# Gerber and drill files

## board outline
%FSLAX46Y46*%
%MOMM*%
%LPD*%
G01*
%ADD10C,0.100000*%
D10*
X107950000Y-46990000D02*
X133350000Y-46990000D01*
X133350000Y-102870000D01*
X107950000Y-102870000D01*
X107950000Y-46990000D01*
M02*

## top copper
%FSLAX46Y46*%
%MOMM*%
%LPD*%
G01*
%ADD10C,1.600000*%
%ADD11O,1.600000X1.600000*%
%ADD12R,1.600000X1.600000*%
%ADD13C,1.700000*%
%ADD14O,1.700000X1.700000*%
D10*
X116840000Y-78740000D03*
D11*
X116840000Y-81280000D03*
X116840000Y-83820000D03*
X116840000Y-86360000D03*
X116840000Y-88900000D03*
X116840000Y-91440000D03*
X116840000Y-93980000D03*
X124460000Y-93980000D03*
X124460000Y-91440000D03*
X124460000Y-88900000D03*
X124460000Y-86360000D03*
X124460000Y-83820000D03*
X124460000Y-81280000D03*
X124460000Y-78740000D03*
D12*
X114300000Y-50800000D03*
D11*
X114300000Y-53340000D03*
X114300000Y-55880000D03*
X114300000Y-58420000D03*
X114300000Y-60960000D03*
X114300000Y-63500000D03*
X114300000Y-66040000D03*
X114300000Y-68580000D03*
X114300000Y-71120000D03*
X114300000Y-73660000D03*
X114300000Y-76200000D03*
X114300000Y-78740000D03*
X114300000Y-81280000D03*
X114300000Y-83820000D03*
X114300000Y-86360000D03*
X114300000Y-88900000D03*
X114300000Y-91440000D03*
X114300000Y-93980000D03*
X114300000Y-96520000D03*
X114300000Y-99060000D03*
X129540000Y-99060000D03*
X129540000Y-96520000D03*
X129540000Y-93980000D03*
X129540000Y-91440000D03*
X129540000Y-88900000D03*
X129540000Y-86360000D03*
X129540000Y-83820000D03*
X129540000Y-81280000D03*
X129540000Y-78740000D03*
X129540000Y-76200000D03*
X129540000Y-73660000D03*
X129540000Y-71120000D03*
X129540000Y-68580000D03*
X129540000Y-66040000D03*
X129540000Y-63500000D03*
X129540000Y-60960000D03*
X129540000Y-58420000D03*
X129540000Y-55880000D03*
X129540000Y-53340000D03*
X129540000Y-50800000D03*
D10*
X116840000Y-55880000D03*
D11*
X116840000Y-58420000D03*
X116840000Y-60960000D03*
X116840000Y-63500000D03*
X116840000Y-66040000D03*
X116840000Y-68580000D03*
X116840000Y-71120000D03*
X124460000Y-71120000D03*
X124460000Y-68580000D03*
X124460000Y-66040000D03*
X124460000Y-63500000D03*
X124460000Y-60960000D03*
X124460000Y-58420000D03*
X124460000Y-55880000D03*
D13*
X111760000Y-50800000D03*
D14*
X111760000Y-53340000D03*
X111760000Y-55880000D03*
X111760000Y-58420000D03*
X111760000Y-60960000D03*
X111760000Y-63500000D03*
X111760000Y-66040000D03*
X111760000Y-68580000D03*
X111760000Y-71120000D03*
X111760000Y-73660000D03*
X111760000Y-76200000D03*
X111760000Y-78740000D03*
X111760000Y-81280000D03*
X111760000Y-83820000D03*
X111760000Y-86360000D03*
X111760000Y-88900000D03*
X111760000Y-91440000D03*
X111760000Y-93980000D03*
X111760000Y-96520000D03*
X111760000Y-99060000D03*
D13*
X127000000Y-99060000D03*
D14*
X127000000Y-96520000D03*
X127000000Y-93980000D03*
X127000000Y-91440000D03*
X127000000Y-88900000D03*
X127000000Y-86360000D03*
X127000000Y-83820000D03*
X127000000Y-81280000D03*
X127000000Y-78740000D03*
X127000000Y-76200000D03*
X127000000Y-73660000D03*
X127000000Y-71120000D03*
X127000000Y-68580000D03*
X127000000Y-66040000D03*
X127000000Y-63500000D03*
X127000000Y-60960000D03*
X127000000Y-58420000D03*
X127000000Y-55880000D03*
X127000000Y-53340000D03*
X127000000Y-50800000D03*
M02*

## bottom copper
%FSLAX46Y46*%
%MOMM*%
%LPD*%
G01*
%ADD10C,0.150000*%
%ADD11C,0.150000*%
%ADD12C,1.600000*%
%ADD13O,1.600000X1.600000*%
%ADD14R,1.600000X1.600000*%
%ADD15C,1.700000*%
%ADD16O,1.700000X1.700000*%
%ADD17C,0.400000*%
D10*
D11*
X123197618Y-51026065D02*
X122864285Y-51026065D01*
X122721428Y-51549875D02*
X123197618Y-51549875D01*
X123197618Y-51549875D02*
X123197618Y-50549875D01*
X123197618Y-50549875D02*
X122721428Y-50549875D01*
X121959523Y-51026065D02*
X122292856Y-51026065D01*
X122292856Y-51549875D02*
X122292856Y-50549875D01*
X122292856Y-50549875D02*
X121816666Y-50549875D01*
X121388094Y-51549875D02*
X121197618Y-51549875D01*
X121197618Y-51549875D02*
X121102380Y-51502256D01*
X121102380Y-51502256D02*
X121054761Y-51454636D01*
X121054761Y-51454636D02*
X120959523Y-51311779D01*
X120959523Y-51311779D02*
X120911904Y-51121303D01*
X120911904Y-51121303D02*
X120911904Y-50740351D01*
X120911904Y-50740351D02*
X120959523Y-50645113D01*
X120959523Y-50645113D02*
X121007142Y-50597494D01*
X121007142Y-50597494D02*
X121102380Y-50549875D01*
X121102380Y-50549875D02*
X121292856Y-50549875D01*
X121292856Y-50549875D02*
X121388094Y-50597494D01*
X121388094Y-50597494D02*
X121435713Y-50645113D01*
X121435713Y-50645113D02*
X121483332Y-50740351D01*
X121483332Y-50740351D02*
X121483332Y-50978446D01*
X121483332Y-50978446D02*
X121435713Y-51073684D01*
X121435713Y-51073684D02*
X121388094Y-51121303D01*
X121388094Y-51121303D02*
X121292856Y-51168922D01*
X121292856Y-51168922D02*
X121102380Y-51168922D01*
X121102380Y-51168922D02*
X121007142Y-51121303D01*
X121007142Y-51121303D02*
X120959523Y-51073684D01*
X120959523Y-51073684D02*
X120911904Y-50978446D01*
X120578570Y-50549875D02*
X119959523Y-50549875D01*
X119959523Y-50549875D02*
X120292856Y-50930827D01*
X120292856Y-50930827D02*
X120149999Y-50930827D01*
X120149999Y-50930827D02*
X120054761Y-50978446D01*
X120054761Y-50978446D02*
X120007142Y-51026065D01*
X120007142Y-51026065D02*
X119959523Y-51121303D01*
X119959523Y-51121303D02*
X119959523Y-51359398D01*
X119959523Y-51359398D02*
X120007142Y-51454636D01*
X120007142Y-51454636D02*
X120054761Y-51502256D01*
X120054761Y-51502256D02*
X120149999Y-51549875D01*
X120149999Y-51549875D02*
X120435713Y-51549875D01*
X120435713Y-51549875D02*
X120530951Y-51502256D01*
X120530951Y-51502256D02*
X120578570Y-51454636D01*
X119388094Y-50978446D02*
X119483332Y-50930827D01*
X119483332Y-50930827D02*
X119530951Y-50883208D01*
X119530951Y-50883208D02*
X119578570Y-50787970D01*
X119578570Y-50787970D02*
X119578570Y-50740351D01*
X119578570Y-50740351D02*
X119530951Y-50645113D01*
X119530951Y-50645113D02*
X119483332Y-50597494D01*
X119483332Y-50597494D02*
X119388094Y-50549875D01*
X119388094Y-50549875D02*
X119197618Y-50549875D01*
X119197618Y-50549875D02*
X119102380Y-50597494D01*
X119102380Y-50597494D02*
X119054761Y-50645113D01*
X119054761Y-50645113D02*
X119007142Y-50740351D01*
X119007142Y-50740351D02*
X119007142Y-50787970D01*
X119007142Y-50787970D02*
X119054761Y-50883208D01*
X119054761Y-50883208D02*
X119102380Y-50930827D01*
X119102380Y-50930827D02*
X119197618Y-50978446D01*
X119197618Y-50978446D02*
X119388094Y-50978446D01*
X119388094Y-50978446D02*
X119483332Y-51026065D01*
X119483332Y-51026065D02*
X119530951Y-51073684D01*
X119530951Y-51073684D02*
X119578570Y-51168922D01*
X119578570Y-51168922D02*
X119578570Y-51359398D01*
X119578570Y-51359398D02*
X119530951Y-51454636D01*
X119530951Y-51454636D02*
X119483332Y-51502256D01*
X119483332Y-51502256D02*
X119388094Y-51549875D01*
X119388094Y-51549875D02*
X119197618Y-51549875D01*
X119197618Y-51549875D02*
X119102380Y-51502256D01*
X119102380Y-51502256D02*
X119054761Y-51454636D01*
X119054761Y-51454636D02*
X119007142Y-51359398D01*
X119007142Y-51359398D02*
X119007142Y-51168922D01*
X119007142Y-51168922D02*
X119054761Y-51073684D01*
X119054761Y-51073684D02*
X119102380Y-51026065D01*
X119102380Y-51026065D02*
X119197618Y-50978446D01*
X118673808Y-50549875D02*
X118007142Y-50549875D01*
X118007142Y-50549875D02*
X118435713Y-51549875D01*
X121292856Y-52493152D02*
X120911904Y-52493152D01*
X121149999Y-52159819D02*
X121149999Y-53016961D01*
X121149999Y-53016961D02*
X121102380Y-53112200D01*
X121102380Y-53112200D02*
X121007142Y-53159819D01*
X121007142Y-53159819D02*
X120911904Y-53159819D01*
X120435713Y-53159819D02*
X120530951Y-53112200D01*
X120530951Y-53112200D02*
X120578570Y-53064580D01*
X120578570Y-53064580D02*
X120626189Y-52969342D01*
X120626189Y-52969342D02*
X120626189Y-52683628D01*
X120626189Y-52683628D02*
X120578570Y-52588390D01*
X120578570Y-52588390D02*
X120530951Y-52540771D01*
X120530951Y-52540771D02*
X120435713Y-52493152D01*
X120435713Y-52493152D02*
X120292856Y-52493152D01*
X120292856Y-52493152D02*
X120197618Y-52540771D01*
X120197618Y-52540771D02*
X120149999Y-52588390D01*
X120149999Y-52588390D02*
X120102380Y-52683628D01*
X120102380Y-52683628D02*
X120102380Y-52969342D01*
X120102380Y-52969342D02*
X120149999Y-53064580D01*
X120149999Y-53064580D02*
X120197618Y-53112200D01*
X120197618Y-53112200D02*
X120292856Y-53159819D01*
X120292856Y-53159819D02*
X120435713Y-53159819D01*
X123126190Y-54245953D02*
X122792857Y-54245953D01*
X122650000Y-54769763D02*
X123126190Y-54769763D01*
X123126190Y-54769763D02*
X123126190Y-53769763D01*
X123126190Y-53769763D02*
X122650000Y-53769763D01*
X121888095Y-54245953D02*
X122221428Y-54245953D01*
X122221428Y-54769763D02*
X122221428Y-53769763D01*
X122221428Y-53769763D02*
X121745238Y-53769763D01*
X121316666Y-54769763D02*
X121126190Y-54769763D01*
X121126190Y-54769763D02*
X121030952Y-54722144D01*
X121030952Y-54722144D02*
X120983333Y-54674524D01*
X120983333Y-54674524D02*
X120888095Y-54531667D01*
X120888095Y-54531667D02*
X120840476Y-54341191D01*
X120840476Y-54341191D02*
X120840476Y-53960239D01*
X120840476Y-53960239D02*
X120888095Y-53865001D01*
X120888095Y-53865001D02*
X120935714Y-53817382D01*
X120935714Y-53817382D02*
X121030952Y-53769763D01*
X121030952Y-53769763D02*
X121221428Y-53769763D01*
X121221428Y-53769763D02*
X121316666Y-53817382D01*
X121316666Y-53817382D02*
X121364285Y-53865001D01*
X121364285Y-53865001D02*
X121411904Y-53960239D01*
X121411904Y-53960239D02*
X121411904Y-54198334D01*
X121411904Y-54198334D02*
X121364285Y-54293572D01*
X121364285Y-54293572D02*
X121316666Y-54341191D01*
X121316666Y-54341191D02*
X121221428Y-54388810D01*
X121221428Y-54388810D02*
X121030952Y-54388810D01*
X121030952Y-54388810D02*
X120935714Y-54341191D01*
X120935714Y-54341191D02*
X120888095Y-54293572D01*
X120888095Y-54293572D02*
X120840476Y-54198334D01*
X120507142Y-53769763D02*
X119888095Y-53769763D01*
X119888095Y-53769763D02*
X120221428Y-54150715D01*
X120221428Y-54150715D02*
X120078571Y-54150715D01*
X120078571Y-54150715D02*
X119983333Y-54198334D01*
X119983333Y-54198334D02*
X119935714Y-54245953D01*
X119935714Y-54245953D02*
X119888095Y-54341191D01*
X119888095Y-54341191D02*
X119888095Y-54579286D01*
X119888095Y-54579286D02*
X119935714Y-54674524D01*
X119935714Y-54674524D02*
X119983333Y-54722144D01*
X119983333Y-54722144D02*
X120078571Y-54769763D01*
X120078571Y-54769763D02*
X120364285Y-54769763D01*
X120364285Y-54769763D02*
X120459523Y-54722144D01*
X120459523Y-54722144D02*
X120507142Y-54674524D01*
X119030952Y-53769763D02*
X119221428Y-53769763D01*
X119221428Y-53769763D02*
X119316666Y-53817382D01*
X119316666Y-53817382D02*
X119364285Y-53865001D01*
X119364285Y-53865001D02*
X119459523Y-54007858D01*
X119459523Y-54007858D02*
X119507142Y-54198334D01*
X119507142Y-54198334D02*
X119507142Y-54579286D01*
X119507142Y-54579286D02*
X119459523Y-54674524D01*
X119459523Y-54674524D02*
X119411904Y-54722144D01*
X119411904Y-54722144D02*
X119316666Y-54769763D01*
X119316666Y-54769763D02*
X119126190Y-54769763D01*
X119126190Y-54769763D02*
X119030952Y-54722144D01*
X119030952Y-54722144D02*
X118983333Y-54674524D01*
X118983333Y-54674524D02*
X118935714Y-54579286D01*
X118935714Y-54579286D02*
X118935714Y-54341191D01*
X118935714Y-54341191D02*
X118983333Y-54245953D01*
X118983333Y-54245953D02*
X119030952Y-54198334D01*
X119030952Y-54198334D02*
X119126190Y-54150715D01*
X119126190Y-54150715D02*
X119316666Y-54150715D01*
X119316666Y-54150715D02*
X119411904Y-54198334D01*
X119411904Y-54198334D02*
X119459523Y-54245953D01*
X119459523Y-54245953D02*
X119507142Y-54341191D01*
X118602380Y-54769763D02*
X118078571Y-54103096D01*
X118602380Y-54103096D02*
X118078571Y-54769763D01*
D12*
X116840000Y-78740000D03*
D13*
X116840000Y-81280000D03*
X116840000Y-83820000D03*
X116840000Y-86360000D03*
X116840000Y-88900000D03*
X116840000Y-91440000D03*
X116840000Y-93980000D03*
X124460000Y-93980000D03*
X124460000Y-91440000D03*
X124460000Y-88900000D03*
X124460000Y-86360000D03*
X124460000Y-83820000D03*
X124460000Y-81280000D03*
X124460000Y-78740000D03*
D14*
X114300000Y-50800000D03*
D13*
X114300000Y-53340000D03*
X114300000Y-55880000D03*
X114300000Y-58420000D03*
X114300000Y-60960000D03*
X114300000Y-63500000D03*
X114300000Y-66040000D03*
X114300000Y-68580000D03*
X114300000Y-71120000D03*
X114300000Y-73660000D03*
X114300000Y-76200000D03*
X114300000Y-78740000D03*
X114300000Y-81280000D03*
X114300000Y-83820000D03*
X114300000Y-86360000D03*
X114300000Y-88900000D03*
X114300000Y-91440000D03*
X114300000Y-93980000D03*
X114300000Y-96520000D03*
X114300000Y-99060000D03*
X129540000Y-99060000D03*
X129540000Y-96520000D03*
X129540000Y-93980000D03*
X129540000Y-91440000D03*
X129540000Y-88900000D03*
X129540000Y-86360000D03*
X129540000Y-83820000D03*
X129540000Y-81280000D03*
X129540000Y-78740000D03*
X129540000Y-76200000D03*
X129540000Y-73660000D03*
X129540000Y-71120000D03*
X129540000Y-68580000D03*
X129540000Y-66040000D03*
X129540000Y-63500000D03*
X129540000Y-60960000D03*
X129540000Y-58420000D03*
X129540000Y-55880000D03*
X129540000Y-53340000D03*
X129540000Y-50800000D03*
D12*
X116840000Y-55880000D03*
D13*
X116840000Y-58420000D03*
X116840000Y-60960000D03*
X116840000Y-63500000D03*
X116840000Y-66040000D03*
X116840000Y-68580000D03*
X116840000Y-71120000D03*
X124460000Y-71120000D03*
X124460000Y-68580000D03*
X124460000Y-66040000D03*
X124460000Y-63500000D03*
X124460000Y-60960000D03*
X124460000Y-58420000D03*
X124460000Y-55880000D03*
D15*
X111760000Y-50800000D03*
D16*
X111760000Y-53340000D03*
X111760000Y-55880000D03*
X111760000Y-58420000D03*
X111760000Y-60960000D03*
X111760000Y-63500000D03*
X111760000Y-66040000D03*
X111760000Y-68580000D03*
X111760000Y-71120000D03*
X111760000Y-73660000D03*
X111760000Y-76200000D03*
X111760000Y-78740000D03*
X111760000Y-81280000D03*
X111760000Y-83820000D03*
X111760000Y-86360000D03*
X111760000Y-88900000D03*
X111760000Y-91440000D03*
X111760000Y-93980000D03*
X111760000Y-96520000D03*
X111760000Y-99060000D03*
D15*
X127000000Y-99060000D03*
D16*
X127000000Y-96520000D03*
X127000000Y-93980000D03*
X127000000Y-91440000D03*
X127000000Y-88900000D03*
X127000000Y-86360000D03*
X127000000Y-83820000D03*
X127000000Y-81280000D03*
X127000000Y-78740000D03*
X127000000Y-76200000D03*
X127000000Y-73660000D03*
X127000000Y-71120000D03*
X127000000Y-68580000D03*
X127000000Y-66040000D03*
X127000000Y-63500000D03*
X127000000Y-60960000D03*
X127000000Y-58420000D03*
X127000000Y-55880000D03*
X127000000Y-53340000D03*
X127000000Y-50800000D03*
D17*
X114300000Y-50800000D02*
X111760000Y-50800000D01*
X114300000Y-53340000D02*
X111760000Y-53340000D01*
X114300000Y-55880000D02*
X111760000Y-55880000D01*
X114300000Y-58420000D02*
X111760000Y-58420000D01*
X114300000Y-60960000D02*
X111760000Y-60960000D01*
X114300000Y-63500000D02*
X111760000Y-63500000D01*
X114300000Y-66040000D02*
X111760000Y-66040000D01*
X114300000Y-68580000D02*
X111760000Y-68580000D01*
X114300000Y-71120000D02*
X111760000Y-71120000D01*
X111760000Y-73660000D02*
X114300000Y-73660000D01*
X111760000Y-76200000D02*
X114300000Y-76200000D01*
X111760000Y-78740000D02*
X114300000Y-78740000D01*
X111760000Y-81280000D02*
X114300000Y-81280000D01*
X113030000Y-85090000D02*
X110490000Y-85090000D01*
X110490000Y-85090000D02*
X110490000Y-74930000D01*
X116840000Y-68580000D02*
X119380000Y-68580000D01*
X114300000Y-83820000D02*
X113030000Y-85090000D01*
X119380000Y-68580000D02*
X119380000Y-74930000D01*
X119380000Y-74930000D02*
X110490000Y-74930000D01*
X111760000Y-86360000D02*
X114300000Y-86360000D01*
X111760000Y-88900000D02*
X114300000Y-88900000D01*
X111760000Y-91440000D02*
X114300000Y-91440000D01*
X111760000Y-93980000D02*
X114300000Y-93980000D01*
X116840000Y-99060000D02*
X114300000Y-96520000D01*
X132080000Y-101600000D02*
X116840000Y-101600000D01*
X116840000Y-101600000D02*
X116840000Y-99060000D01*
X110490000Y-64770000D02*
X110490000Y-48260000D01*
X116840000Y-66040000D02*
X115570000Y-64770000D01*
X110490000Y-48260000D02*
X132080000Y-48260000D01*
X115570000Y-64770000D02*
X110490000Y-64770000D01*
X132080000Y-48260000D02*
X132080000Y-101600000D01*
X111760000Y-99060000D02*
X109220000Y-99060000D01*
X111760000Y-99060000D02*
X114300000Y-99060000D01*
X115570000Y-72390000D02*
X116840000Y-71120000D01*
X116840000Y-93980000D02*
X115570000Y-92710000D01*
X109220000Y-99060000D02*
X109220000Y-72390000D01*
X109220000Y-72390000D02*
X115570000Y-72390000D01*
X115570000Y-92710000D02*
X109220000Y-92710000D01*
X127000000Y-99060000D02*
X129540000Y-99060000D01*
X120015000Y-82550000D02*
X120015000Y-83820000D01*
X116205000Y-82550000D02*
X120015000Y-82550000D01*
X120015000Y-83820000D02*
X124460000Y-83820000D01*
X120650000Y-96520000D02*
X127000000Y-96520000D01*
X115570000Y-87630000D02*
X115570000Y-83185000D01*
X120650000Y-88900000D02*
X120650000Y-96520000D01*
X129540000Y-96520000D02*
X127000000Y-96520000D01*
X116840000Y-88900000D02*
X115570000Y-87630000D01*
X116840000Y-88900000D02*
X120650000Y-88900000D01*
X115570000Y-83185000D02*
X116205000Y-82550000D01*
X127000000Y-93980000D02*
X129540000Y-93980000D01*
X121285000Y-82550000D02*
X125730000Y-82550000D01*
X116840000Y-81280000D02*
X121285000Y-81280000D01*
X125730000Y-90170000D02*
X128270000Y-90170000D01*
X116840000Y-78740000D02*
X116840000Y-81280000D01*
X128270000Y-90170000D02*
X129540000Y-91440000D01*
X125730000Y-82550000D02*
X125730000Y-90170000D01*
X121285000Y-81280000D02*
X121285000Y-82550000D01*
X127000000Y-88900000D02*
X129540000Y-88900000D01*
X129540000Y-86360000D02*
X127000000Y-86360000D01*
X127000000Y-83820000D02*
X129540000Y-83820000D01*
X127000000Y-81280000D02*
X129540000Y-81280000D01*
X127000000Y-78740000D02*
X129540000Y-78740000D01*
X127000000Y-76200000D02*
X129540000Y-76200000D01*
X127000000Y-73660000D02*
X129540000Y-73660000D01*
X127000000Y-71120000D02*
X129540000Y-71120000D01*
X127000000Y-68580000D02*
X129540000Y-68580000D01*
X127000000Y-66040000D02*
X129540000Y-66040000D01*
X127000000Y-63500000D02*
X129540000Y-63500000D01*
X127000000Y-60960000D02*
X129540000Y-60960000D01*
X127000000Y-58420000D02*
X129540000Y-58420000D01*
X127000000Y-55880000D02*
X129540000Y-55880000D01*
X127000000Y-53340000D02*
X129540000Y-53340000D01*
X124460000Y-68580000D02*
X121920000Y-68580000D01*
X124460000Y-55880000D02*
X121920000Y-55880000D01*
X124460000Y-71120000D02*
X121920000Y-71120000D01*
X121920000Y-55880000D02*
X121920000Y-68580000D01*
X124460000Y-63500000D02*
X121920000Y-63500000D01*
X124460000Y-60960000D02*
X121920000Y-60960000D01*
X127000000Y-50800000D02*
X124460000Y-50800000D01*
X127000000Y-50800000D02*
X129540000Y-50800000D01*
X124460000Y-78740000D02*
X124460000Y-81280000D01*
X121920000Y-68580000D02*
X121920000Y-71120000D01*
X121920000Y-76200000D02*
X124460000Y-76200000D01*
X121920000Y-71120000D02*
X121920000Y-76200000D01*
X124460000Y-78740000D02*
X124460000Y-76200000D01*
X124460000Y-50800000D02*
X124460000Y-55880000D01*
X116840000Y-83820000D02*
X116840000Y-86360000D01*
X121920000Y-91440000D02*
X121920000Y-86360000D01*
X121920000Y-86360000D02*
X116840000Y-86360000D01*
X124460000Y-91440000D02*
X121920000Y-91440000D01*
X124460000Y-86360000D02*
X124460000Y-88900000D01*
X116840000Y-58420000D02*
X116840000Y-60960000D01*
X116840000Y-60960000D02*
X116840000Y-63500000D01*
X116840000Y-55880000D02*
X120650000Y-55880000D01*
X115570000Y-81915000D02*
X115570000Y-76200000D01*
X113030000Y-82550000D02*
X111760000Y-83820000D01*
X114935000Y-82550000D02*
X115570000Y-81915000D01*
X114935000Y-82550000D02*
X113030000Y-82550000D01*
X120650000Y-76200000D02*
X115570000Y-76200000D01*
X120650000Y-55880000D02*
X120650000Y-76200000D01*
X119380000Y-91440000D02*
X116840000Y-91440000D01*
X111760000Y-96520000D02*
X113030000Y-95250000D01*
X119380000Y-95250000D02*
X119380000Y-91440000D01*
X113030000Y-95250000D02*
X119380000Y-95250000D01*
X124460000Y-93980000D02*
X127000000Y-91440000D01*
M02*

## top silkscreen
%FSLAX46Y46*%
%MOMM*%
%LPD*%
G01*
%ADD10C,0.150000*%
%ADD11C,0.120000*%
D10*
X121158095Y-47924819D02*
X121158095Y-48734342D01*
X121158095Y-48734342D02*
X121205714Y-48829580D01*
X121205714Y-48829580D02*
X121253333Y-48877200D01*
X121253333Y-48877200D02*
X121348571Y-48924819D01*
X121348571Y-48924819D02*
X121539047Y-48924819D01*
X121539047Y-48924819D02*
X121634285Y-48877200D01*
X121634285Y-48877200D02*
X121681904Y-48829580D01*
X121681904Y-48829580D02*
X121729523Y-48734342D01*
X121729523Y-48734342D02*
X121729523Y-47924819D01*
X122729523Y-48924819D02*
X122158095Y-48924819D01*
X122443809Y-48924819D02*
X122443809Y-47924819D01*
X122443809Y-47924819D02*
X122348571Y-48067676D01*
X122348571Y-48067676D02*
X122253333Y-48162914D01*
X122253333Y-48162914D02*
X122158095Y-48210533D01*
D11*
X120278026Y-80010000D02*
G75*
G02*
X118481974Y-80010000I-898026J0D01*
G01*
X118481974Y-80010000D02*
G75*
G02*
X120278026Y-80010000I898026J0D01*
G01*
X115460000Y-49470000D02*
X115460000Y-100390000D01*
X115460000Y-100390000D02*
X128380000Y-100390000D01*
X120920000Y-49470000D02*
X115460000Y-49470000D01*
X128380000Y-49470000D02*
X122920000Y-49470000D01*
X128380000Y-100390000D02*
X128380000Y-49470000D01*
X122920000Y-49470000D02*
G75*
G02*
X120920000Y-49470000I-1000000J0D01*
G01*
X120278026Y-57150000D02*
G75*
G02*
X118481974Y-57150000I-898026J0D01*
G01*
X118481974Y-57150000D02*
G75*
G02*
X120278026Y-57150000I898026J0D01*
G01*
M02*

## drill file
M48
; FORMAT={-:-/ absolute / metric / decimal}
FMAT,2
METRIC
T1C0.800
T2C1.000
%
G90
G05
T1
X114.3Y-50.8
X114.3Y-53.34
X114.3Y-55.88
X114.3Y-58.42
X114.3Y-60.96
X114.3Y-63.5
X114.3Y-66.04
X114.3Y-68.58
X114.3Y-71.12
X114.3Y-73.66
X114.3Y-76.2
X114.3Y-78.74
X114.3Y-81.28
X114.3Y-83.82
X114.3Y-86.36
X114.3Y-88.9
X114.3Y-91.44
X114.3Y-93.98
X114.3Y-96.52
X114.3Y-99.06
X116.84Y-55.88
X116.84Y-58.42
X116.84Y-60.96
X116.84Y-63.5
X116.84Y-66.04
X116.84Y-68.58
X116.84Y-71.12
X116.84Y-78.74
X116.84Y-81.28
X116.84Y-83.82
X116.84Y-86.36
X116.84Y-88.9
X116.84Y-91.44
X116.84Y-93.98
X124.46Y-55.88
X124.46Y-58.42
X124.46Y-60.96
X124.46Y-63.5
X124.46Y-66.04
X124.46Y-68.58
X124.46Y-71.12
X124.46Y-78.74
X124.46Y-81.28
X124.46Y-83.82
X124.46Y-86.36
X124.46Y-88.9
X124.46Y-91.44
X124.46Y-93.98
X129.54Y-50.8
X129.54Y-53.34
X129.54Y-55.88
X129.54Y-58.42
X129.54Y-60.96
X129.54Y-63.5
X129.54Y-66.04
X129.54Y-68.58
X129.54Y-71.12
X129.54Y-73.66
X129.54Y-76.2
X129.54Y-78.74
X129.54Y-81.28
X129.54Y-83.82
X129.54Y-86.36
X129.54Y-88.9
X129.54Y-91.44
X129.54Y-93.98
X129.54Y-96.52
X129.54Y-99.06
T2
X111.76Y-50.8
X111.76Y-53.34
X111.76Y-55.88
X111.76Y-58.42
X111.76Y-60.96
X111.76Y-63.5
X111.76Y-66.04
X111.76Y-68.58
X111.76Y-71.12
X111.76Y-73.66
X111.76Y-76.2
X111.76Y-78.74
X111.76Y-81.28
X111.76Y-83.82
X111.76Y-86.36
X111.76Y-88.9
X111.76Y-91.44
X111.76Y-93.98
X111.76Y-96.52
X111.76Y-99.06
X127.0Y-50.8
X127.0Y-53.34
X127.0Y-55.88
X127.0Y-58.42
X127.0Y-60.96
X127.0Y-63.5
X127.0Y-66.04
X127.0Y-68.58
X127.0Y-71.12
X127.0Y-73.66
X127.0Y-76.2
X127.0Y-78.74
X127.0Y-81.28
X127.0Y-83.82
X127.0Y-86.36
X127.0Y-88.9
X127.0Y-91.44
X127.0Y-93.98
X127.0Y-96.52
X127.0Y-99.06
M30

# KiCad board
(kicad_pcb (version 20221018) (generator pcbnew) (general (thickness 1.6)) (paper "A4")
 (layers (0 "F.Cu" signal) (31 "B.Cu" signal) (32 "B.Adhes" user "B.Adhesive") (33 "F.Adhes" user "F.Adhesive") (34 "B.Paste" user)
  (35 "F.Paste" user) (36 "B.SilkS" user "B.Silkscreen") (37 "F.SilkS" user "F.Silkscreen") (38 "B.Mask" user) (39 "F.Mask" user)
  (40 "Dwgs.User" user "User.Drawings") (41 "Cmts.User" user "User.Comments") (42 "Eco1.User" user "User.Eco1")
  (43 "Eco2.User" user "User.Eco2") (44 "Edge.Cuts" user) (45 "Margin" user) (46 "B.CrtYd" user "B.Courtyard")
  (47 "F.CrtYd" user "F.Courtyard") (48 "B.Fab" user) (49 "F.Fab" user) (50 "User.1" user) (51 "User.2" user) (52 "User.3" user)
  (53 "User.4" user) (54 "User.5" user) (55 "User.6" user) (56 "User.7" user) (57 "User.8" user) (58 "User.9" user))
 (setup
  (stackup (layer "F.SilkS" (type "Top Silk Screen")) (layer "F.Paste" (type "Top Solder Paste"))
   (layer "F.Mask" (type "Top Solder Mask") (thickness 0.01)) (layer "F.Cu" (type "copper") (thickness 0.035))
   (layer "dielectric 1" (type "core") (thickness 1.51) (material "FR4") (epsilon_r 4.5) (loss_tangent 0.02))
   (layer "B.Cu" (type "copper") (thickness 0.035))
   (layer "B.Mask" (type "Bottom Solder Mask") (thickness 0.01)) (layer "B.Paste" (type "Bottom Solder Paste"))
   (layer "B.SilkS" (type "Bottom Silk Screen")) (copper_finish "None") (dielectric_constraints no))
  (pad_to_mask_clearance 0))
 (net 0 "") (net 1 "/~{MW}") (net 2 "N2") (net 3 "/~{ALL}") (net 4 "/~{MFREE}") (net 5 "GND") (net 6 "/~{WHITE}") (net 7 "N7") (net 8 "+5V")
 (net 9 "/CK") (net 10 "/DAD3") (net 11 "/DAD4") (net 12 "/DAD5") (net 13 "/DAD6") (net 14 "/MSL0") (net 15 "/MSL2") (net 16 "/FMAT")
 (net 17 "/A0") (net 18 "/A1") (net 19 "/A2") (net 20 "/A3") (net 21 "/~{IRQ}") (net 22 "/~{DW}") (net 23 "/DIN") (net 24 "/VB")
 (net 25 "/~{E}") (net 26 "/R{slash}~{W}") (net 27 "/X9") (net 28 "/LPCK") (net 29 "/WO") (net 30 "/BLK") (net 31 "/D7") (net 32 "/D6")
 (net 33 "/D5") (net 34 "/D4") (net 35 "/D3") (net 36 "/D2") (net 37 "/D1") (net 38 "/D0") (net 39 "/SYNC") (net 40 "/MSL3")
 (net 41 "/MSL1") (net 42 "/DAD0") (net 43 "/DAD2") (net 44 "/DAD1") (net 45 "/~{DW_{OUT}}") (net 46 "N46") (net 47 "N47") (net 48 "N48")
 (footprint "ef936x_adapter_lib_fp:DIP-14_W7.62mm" (layer "F.Cu") (at 116.84 78.74)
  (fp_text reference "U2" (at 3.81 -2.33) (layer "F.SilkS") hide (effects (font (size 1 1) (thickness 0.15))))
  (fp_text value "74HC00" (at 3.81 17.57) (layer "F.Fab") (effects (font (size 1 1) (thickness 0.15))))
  (fp_circle (center 2.54 1.27) (end 3.438026 1.27) (stroke (width 0.12) (type solid)) (fill none) (layer "F.SilkS"))
  (pad "1" thru_hole circle (at 0 0) (size 1.6 1.6) (drill 0.8) (layers "*.Cu" "*.Mask") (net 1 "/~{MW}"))
  (pad "2" thru_hole oval (at 0 2.54) (size 1.6 1.6) (drill 0.8) (layers "*.Cu" "*.Mask") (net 1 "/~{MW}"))
  (pad "3" thru_hole oval (at 0 5.08) (size 1.6 1.6) (drill 0.8) (layers "*.Cu" "*.Mask") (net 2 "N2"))
  (pad "4" thru_hole oval (at 0 7.62) (size 1.6 1.6) (drill 0.8) (layers "*.Cu" "*.Mask") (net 2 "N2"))
  (pad "5" thru_hole oval (at 0 10.16) (size 1.6 1.6) (drill 0.8) (layers "*.Cu" "*.Mask") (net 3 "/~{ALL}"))
  (pad "6" thru_hole oval (at 0 12.7) (size 1.6 1.6) (drill 0.8) (layers "*.Cu" "*.Mask") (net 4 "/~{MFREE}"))
  (pad "7" thru_hole oval (at 0 15.24) (size 1.6 1.6) (drill 0.8) (layers "*.Cu" "*.Mask") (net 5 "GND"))
  (pad "8" thru_hole oval (at 7.62 15.24) (size 1.6 1.6) (drill 0.8) (layers "*.Cu" "*.Mask") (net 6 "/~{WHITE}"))
  (pad "9" thru_hole oval (at 7.62 12.7) (size 1.6 1.6) (drill 0.8) (layers "*.Cu" "*.Mask") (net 2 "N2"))
  (pad "10" thru_hole oval (at 7.62 10.16) (size 1.6 1.6) (drill 0.8) (layers "*.Cu" "*.Mask") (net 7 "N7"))
  (pad "11" thru_hole oval (at 7.62 7.62) (size 1.6 1.6) (drill 0.8) (layers "*.Cu" "*.Mask") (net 7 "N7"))
  (pad "12" thru_hole oval (at 7.62 5.08) (size 1.6 1.6) (drill 0.8) (layers "*.Cu" "*.Mask") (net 3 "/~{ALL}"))
  (pad "13" thru_hole oval (at 7.62 2.54) (size 1.6 1.6) (drill 0.8) (layers "*.Cu" "*.Mask") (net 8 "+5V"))
  (pad "14" thru_hole oval (at 7.62 0) (size 1.6 1.6) (drill 0.8) (layers "*.Cu" "*.Mask") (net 8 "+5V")))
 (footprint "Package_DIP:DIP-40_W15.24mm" (layer "F.Cu") (at 114.3 50.8)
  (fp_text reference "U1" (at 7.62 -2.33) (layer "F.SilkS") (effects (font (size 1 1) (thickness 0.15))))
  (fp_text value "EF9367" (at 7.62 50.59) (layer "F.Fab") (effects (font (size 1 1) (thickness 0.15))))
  (fp_line (start 1.16 -1.33) (end 1.16 49.59) (stroke (width 0.12) (type solid)) (layer "F.SilkS"))
  (fp_line (start 1.16 49.59) (end 14.08 49.59) (stroke (width 0.12) (type solid)) (layer "F.SilkS"))
  (fp_line (start 6.62 -1.33) (end 1.16 -1.33) (stroke (width 0.12) (type solid)) (layer "F.SilkS"))
  (fp_line (start 14.08 -1.33) (end 8.62 -1.33) (stroke (width 0.12) (type solid)) (layer "F.SilkS"))
  (fp_line (start 14.08 49.59) (end 14.08 -1.33) (stroke (width 0.12) (type solid)) (layer "F.SilkS"))
  (fp_arc (start 8.62 -1.33) (mid 7.62 -0.33) (end 6.62 -1.33) (stroke (width 0.12) (type solid)) (layer "F.SilkS"))
  (pad "1" thru_hole rect (at 0 0) (size 1.6 1.6) (drill 0.8) (layers "*.Cu" "*.Mask") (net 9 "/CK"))
  (pad "2" thru_hole oval (at 0 2.54) (size 1.6 1.6) (drill 0.8) (layers "*.Cu" "*.Mask") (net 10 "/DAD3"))
  (pad "3" thru_hole oval (at 0 5.08) (size 1.6 1.6) (drill 0.8) (layers "*.Cu" "*.Mask") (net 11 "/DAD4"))
  (pad "4" thru_hole oval (at 0 7.62) (size 1.6 1.6) (drill 0.8) (layers "*.Cu" "*.Mask") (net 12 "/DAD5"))
  (pad "5" thru_hole oval (at 0 10.16) (size 1.6 1.6) (drill 0.8) (layers "*.Cu" "*.Mask") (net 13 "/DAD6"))
  (pad "6" thru_hole oval (at 0 12.7) (size 1.6 1.6) (drill 0.8) (layers "*.Cu" "*.Mask") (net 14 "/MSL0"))
  (pad "7" thru_hole oval (at 0 15.24) (size 1.6 1.6) (drill 0.8) (layers "*.Cu" "*.Mask") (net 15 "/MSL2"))
  (pad "8" thru_hole oval (at 0 17.78) (size 1.6 1.6) (drill 0.8) (layers "*.Cu" "*.Mask") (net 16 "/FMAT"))
  (pad "9" thru_hole oval (at 0 20.32) (size 1.6 1.6) (drill 0.8) (layers "*.Cu" "*.Mask") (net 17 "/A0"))
  (pad "10" thru_hole oval (at 0 22.86) (size 1.6 1.6) (drill 0.8) (layers "*.Cu" "*.Mask") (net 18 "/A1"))
  (pad "11" thru_hole oval (at 0 25.4) (size 1.6 1.6) (drill 0.8) (layers "*.Cu" "*.Mask") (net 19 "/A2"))
  (pad "12" thru_hole oval (at 0 27.94) (size 1.6 1.6) (drill 0.8) (layers "*.Cu" "*.Mask") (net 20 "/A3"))
  (pad "13" thru_hole oval (at 0 30.48) (size 1.6 1.6) (drill 0.8) (layers "*.Cu" "*.Mask") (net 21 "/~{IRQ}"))
  (pad "14" thru_hole oval (at 0 33.02) (size 1.6 1.6) (drill 0.8) (layers "*.Cu" "*.Mask") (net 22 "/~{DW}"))
  (pad "15" thru_hole oval (at 0 35.56) (size 1.6 1.6) (drill 0.8) (layers "*.Cu" "*.Mask") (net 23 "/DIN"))
  (pad "16" thru_hole oval (at 0 38.1) (size 1.6 1.6) (drill 0.8) (layers "*.Cu" "*.Mask") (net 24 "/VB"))
  (pad "17" thru_hole oval (at 0 40.64) (size 1.6 1.6) (drill 0.8) (layers "*.Cu" "*.Mask") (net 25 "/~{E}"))
  (pad "18" thru_hole oval (at 0 43.18) (size 1.6 1.6) (drill 0.8) (layers "*.Cu" "*.Mask") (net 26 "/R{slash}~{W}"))
  (pad "19" thru_hole oval (at 0 45.72) (size 1.6 1.6) (drill 0.8) (layers "*.Cu" "*.Mask") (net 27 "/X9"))
  (pad "20" thru_hole oval (at 0 48.26) (size 1.6 1.6) (drill 0.8) (layers "*.Cu" "*.Mask") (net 5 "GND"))
  (pad "21" thru_hole oval (at 15.24 48.26) (size 1.6 1.6) (drill 0.8) (layers "*.Cu" "*.Mask") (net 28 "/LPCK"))
  (pad "22" thru_hole oval (at 15.24 45.72) (size 1.6 1.6) (drill 0.8) (layers "*.Cu" "*.Mask") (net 3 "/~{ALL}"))
  (pad "23" thru_hole oval (at 15.24 43.18) (size 1.6 1.6) (drill 0.8) (layers "*.Cu" "*.Mask") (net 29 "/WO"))
  (pad "24" thru_hole oval (at 15.24 40.64) (size 1.6 1.6) (drill 0.8) (layers "*.Cu" "*.Mask") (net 1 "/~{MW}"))
  (pad "25" thru_hole oval (at 15.24 38.1) (size 1.6 1.6) (drill 0.8) (layers "*.Cu" "*.Mask") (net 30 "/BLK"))
  (pad "26" thru_hole oval (at 15.24 35.56) (size 1.6 1.6) (drill 0.8) (layers "*.Cu" "*.Mask") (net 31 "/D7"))
  (pad "27" thru_hole oval (at 15.24 33.02) (size 1.6 1.6) (drill 0.8) (layers "*.Cu" "*.Mask") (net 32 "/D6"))
  (pad "28" thru_hole oval (at 15.24 30.48) (size 1.6 1.6) (drill 0.8) (layers "*.Cu" "*.Mask") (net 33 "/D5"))
  (pad "29" thru_hole oval (at 15.24 27.94) (size 1.6 1.6) (drill 0.8) (layers "*.Cu" "*.Mask") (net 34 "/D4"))
  (pad "30" thru_hole oval (at 15.24 25.4) (size 1.6 1.6) (drill 0.8) (layers "*.Cu" "*.Mask") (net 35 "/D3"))
  (pad "31" thru_hole oval (at 15.24 22.86) (size 1.6 1.6) (drill 0.8) (layers "*.Cu" "*.Mask") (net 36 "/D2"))
  (pad "32" thru_hole oval (at 15.24 20.32) (size 1.6 1.6) (drill 0.8) (layers "*.Cu" "*.Mask") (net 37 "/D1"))
  (pad "33" thru_hole oval (at 15.24 17.78) (size 1.6 1.6) (drill 0.8) (layers "*.Cu" "*.Mask") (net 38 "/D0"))
  (pad "34" thru_hole oval (at 15.24 15.24) (size 1.6 1.6) (drill 0.8) (layers "*.Cu" "*.Mask") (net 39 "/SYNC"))
  (pad "35" thru_hole oval (at 15.24 12.7) (size 1.6 1.6) (drill 0.8) (layers "*.Cu" "*.Mask") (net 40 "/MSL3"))
  (pad "36" thru_hole oval (at 15.24 10.16) (size 1.6 1.6) (drill 0.8) (layers "*.Cu" "*.Mask") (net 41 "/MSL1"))
  (pad "37" thru_hole oval (at 15.24 7.62) (size 1.6 1.6) (drill 0.8) (layers "*.Cu" "*.Mask") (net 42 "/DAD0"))
  (pad "38" thru_hole oval (at 15.24 5.08) (size 1.6 1.6) (drill 0.8) (layers "*.Cu" "*.Mask") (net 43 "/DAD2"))
  (pad "39" thru_hole oval (at 15.24 2.54) (size 1.6 1.6) (drill 0.8) (layers "*.Cu" "*.Mask") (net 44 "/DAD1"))
  (pad "40" thru_hole oval (at 15.24 0) (size 1.6 1.6) (drill 0.8) (layers "*.Cu" "*.Mask") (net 8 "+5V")))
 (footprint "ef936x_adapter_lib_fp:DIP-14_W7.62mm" (layer "F.Cu") (at 116.84 55.88)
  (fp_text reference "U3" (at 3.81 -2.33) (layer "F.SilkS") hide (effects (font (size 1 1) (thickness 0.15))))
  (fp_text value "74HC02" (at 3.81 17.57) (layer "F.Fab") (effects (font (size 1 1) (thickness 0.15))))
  (fp_circle (center 2.54 1.27) (end 3.438026 1.27) (stroke (width 0.12) (type solid)) (fill none) (layer "F.SilkS"))
  (pad "1" thru_hole circle (at 0 0) (size 1.6 1.6) (drill 0.8) (layers "*.Cu" "*.Mask") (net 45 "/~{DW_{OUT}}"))
  (pad "2" thru_hole oval (at 0 2.54) (size 1.6 1.6) (drill 0.8) (layers "*.Cu" "*.Mask") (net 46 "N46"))
  (pad "3" thru_hole oval (at 0 5.08) (size 1.6 1.6) (drill 0.8) (layers "*.Cu" "*.Mask") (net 46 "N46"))
  (pad "4" thru_hole oval (at 0 7.62) (size 1.6 1.6) (drill 0.8) (layers "*.Cu" "*.Mask") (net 46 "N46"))
  (pad "5" thru_hole oval (at 0 10.16) (size 1.6 1.6) (drill 0.8) (layers "*.Cu" "*.Mask") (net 27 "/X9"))
  (pad "6" thru_hole oval (at 0 12.7) (size 1.6 1.6) (drill 0.8) (layers "*.Cu" "*.Mask") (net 22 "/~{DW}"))
  (pad "7" thru_hole oval (at 0 15.24) (size 1.6 1.6) (drill 0.8) (layers "*.Cu" "*.Mask") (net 5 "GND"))
  (pad "8" thru_hole oval (at 7.62 15.24) (size 1.6 1.6) (drill 0.8) (layers "*.Cu" "*.Mask") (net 8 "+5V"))
  (pad "9" thru_hole oval (at 7.62 12.7) (size 1.6 1.6) (drill 0.8) (layers "*.Cu" "*.Mask") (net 8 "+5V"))
  (pad "10" thru_hole oval (at 7.62 10.16) (size 1.6 1.6) (drill 0.8) (layers "*.Cu" "*.Mask") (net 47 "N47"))
  (pad "11" thru_hole oval (at 7.62 7.62) (size 1.6 1.6) (drill 0.8) (layers "*.Cu" "*.Mask") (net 8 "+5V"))
  (pad "12" thru_hole oval (at 7.62 5.08) (size 1.6 1.6) (drill 0.8) (layers "*.Cu" "*.Mask") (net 8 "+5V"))
  (pad "13" thru_hole oval (at 7.62 2.54) (size 1.6 1.6) (drill 0.8) (layers "*.Cu" "*.Mask") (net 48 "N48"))
  (pad "14" thru_hole oval (at 7.62 0) (size 1.6 1.6) (drill 0.8) (layers "*.Cu" "*.Mask") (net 8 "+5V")))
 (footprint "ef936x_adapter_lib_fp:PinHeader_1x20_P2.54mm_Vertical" (layer "B.Cu") (at 111.76 50.8 180)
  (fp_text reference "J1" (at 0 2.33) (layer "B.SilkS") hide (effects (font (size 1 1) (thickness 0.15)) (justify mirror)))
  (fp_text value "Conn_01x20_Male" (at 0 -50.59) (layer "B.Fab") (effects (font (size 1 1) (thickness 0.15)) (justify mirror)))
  (pad "1" thru_hole circle (at 0 0 180) (size 1.7 1.7) (drill 1) (layers "*.Cu" "*.Mask") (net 9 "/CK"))
  (pad "2" thru_hole oval (at 0 -2.54 180) (size 1.7 1.7) (drill 1) (layers "*.Cu" "*.Mask") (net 10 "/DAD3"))
  (pad "3" thru_hole oval (at 0 -5.08 180) (size 1.7 1.7) (drill 1) (layers "*.Cu" "*.Mask") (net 11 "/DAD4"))
  (pad "4" thru_hole oval (at 0 -7.62 180) (size 1.7 1.7) (drill 1) (layers "*.Cu" "*.Mask") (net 12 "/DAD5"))
  (pad "5" thru_hole oval (at 0 -10.16 180) (size 1.7 1.7) (drill 1) (layers "*.Cu" "*.Mask") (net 13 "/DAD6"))
  (pad "6" thru_hole oval (at 0 -12.7 180) (size 1.7 1.7) (drill 1) (layers "*.Cu" "*.Mask") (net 14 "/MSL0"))
  (pad "7" thru_hole oval (at 0 -15.24 180) (size 1.7 1.7) (drill 1) (layers "*.Cu" "*.Mask") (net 15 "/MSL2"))
  (pad "8" thru_hole oval (at 0 -17.78 180) (size 1.7 1.7) (drill 1) (layers "*.Cu" "*.Mask") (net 16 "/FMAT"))
  (pad "9" thru_hole oval (at 0 -20.32 180) (size 1.7 1.7) (drill 1) (layers "*.Cu" "*.Mask") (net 17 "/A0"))
  (pad "10" thru_hole oval (at 0 -22.86 180) (size 1.7 1.7) (drill 1) (layers "*.Cu" "*.Mask") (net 18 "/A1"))
  (pad "11" thru_hole oval (at 0 -25.4 180) (size 1.7 1.7) (drill 1) (layers "*.Cu" "*.Mask") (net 19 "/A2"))
  (pad "12" thru_hole oval (at 0 -27.94 180) (size 1.7 1.7) (drill 1) (layers "*.Cu" "*.Mask") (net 20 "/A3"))
  (pad "13" thru_hole oval (at 0 -30.48 180) (size 1.7 1.7) (drill 1) (layers "*.Cu" "*.Mask") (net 21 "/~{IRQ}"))
  (pad "14" thru_hole oval (at 0 -33.02 180) (size 1.7 1.7) (drill 1) (layers "*.Cu" "*.Mask") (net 45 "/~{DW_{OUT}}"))
  (pad "15" thru_hole oval (at 0 -35.56 180) (size 1.7 1.7) (drill 1) (layers "*.Cu" "*.Mask") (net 23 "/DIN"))
  (pad "16" thru_hole oval (at 0 -38.1 180) (size 1.7 1.7) (drill 1) (layers "*.Cu" "*.Mask") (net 24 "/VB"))
  (pad "17" thru_hole oval (at 0 -40.64 180) (size 1.7 1.7) (drill 1) (layers "*.Cu" "*.Mask") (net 25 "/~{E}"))
  (pad "18" thru_hole oval (at 0 -43.18 180) (size 1.7 1.7) (drill 1) (layers "*.Cu" "*.Mask") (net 26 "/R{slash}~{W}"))
  (pad "19" thru_hole oval (at 0 -45.72 180) (size 1.7 1.7) (drill 1) (layers "*.Cu" "*.Mask") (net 4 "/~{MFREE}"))
  (pad "20" thru_hole oval (at 0 -48.26 180) (size 1.7 1.7) (drill 1) (layers "*.Cu" "*.Mask") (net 5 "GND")))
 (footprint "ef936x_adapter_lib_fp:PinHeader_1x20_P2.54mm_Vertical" (layer "B.Cu") (at 127 99.06)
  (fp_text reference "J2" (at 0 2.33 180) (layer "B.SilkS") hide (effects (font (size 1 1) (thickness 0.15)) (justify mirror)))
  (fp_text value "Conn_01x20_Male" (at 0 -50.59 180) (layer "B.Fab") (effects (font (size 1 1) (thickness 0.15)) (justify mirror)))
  (pad "1" thru_hole circle (at 0 0) (size 1.7 1.7) (drill 1) (layers "*.Cu" "*.Mask") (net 28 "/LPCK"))
  (pad "2" thru_hole oval (at 0 -2.54) (size 1.7 1.7) (drill 1) (layers "*.Cu" "*.Mask") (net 3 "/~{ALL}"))
  (pad "3" thru_hole oval (at 0 -5.08) (size 1.7 1.7) (drill 1) (layers "*.Cu" "*.Mask") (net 29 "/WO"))
  (pad "4" thru_hole oval (at 0 -7.62) (size 1.7 1.7) (drill 1) (layers "*.Cu" "*.Mask") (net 6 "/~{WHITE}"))
  (pad "5" thru_hole oval (at 0 -10.16) (size 1.7 1.7) (drill 1) (layers "*.Cu" "*.Mask") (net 30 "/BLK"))
  (pad "6" thru_hole oval (at 0 -12.7) (size 1.7 1.7) (drill 1) (layers "*.Cu" "*.Mask") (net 31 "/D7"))
  (pad "7" thru_hole oval (at 0 -15.24) (size 1.7 1.7) (drill 1) (layers "*.Cu" "*.Mask") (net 32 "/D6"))
  (pad "8" thru_hole oval (at 0 -17.78) (size 1.7 1.7) (drill 1) (layers "*.Cu" "*.Mask") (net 33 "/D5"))
  (pad "9" thru_hole oval (at 0 -20.32) (size 1.7 1.7) (drill 1) (layers "*.Cu" "*.Mask") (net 34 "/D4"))
  (pad "10" thru_hole oval (at 0 -22.86) (size 1.7 1.7) (drill 1) (layers "*.Cu" "*.Mask") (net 35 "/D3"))
  (pad "11" thru_hole oval (at 0 -25.4) (size 1.7 1.7) (drill 1) (layers "*.Cu" "*.Mask") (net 36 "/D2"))
  (pad "12" thru_hole oval (at 0 -27.94) (size 1.7 1.7) (drill 1) (layers "*.Cu" "*.Mask") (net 37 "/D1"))
  (pad "13" thru_hole oval (at 0 -30.48) (size 1.7 1.7) (drill 1) (layers "*.Cu" "*.Mask") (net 38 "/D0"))
  (pad "14" thru_hole oval (at 0 -33.02) (size 1.7 1.7) (drill 1) (layers "*.Cu" "*.Mask") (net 39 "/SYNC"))
  (pad "15" thru_hole oval (at 0 -35.56) (size 1.7 1.7) (drill 1) (layers "*.Cu" "*.Mask") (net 40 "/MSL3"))
  (pad "16" thru_hole oval (at 0 -38.1) (size 1.7 1.7) (drill 1) (layers "*.Cu" "*.Mask") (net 41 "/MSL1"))
  (pad "17" thru_hole oval (at 0 -40.64) (size 1.7 1.7) (drill 1) (layers "*.Cu" "*.Mask") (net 42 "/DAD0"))
  (pad "18" thru_hole oval (at 0 -43.18) (size 1.7 1.7) (drill 1) (layers "*.Cu" "*.Mask") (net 43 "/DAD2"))
  (pad "19" thru_hole oval (at 0 -45.72) (size 1.7 1.7) (drill 1) (layers "*.Cu" "*.Mask") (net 44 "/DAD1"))
  (pad "20" thru_hole oval (at 0 -48.26) (size 1.7 1.7) (drill 1) (layers "*.Cu" "*.Mask") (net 8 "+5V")))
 (gr_rect (start 107.95 46.99) (end 133.35 102.87) (stroke (width 0.1) (type solid)) (fill none) (layer "Edge.Cuts"))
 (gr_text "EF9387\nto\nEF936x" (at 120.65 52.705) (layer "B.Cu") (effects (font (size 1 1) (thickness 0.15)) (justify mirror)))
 (segment (start 114.3 50.8) (end 111.76 50.8) (width 0.4) (layer "B.Cu") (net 9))
 (segment (start 114.3 53.34) (end 111.76 53.34) (width 0.4) (layer "B.Cu") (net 10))
 (segment (start 114.3 55.88) (end 111.76 55.88) (width 0.4) (layer "B.Cu") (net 11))
 (segment (start 114.3 58.42) (end 111.76 58.42) (width 0.4) (layer "B.Cu") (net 12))
 (segment (start 114.3 60.96) (end 111.76 60.96) (width 0.4) (layer "B.Cu") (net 13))
 (segment (start 114.3 63.5) (end 111.76 63.5) (width 0.4) (layer "B.Cu") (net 14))
 (segment (start 114.3 66.04) (end 111.76 66.04) (width 0.4) (layer "B.Cu") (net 15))
 (segment (start 114.3 68.58) (end 111.76 68.58) (width 0.4) (layer "B.Cu") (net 16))
 (segment (start 114.3 71.12) (end 111.76 71.12) (width 0.4) (layer "B.Cu") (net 17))
 (segment (start 111.76 73.66) (end 114.3 73.66) (width 0.4) (layer "B.Cu") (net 18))
 (segment (start 111.76 76.2) (end 114.3 76.2) (width 0.4) (layer "B.Cu") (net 19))
 (segment (start 111.76 78.74) (end 114.3 78.74) (width 0.4) (layer "B.Cu") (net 20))
 (segment (start 111.76 81.28) (end 114.3 81.28) (width 0.4) (layer "B.Cu") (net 21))
 (segment (start 113.03 85.09) (end 110.49 85.09) (width 0.4) (layer "B.Cu") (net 22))
 (segment (start 110.49 85.09) (end 110.49 74.93) (width 0.4) (layer "B.Cu") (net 22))
 (segment (start 116.84 68.58) (end 119.38 68.58) (width 0.4) (layer "B.Cu") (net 22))
 (segment (start 114.3 83.82) (end 113.03 85.09) (width 0.4) (layer "B.Cu") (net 22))
 (segment (start 119.38 68.58) (end 119.38 74.93) (width 0.4) (layer "B.Cu") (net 22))
 (segment (start 119.38 74.93) (end 110.49 74.93) (width 0.4) (layer "B.Cu") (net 22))
 (segment (start 111.76 86.36) (end 114.3 86.36) (width 0.4) (layer "B.Cu") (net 23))
 (segment (start 111.76 88.9) (end 114.3 88.9) (width 0.4) (layer "B.Cu") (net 24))
 (segment (start 111.76 91.44) (end 114.3 91.44) (width 0.4) (layer "B.Cu") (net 25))
 (segment (start 111.76 93.98) (end 114.3 93.98) (width 0.4) (layer "B.Cu") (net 26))
 (segment (start 116.84 99.06) (end 114.3 96.52) (width 0.4) (layer "B.Cu") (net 27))
 (segment (start 132.08 101.6) (end 116.84 101.6) (width 0.4) (layer "B.Cu") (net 27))
 (segment (start 116.84 101.6) (end 116.84 99.06) (width 0.4) (layer "B.Cu") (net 27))
 (segment (start 110.49 64.77) (end 110.49 48.26) (width 0.4) (layer "B.Cu") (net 27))
 (segment (start 116.84 66.04) (end 115.57 64.77) (width 0.4) (layer "B.Cu") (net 27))
 (segment (start 110.49 48.26) (end 132.08 48.26) (width 0.4) (layer "B.Cu") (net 27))
 (segment (start 115.57 64.77) (end 110.49 64.77) (width 0.4) (layer "B.Cu") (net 27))
 (segment (start 132.08 48.26) (end 132.08 101.6) (width 0.4) (layer "B.Cu") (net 27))
 (segment (start 111.76 99.06) (end 109.22 99.06) (width 0.4) (layer "B.Cu") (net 5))
 (segment (start 111.76 99.06) (end 114.3 99.06) (width 0.4) (layer "B.Cu") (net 5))
 (segment (start 115.57 72.39) (end 116.84 71.12) (width 0.4) (layer "B.Cu") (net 5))
 (segment (start 116.84 93.98) (end 115.57 92.71) (width 0.4) (layer "B.Cu") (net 5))
 (segment (start 109.22 99.06) (end 109.22 72.39) (width 0.4) (layer "B.Cu") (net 5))
 (segment (start 109.22 72.39) (end 115.57 72.39) (width 0.4) (layer "B.Cu") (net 5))
 (segment (start 115.57 92.71) (end 109.22 92.71) (width 0.4) (layer "B.Cu") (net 5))
 (segment (start 127 99.06) (end 129.54 99.06) (width 0.4) (layer "B.Cu") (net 28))
 (segment (start 120.015 82.55) (end 120.015 83.82) (width 0.4) (layer "B.Cu") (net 3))
 (segment (start 116.205 82.55) (end 120.015 82.55) (width 0.4) (layer "B.Cu") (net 3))
 (segment (start 120.015 83.82) (end 124.46 83.82) (width 0.4) (layer "B.Cu") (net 3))
 (segment (start 120.65 96.52) (end 127 96.52) (width 0.4) (layer "B.Cu") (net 3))
 (segment (start 115.57 87.63) (end 115.57 83.185) (width 0.4) (layer "B.Cu") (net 3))
 (segment (start 120.65 88.9) (end 120.65 96.52) (width 0.4) (layer "B.Cu") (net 3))
 (segment (start 129.54 96.52) (end 127 96.52) (width 0.4) (layer "B.Cu") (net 3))
 (segment (start 116.84 88.9) (end 115.57 87.63) (width 0.4) (layer "B.Cu") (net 3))
 (segment (start 116.84 88.9) (end 120.65 88.9) (width 0.4) (layer "B.Cu") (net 3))
 (segment (start 115.57 83.185) (end 116.205 82.55) (width 0.4) (layer "B.Cu") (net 3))
 (segment (start 127 93.98) (end 129.54 93.98) (width 0.4) (layer "B.Cu") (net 29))
 (segment (start 121.285 82.55) (end 125.73 82.55) (width 0.4) (layer "B.Cu") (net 1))
 (segment (start 116.84 81.28) (end 121.285 81.28) (width 0.4) (layer "B.Cu") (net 1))
 (segment (start 125.73 90.17) (end 128.27 90.17) (width 0.4) (layer "B.Cu") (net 1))
 (segment (start 116.84 78.74) (end 116.84 81.28) (width 0.4) (layer "B.Cu") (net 1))
 (segment (start 128.27 90.17) (end 129.54 91.44) (width 0.4) (layer "B.Cu") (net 1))
 (segment (start 125.73 82.55) (end 125.73 90.17) (width 0.4) (layer "B.Cu") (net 1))
 (segment (start 121.285 81.28) (end 121.285 82.55) (width 0.4) (layer "B.Cu") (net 1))
 (segment (start 127 88.9) (end 129.54 88.9) (width 0.4) (layer "B.Cu") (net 30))
 (segment (start 129.54 86.36) (end 127 86.36) (width 0.4) (layer "B.Cu") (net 31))
 (segment (start 127 83.82) (end 129.54 83.82) (width 0.4) (layer "B.Cu") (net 32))
 (segment (start 127 81.28) (end 129.54 81.28) (width 0.4) (layer "B.Cu") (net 33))
 (segment (start 127 78.74) (end 129.54 78.74) (width 0.4) (layer "B.Cu") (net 34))
 (segment (start 127 76.2) (end 129.54 76.2) (width 0.4) (layer "B.Cu") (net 35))
 (segment (start 127 73.66) (end 129.54 73.66) (width 0.4) (layer "B.Cu") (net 36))
 (segment (start 127 71.12) (end 129.54 71.12) (width 0.4) (layer "B.Cu") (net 37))
 (segment (start 127 68.58) (end 129.54 68.58) (width 0.4) (layer "B.Cu") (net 38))
 (segment (start 127 66.04) (end 129.54 66.04) (width 0.4) (layer "B.Cu") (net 39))
 (segment (start 127 63.5) (end 129.54 63.5) (width 0.4) (layer "B.Cu") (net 40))
 (segment (start 127 60.96) (end 129.54 60.96) (width 0.4) (layer "B.Cu") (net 41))
 (segment (start 127 58.42) (end 129.54 58.42) (width 0.4) (layer "B.Cu") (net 42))
 (segment (start 127 55.88) (end 129.54 55.88) (width 0.4) (layer "B.Cu") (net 43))
 (segment (start 127 53.34) (end 129.54 53.34) (width 0.4) (layer "B.Cu") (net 44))
 (segment (start 124.46 68.58) (end 121.92 68.58) (width 0.4) (layer "B.Cu") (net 8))
 (segment (start 124.46 55.88) (end 121.92 55.88) (width 0.4) (layer "B.Cu") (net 8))
 (segment (start 124.46 71.12) (end 121.92 71.12) (width 0.4) (layer "B.Cu") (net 8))
 (segment (start 121.92 55.88) (end 121.92 68.58) (width 0.4) (layer "B.Cu") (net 8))
 (segment (start 124.46 63.5) (end 121.92 63.5) (width 0.4) (layer "B.Cu") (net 8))
 (segment (start 124.46 60.96) (end 121.92 60.96) (width 0.4) (layer "B.Cu") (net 8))
 (segment (start 127 50.8) (end 124.46 50.8) (width 0.4) (layer "B.Cu") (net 8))
 (segment (start 127 50.8) (end 129.54 50.8) (width 0.4) (layer "B.Cu") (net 8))
 (segment (start 124.46 78.74) (end 124.46 81.28) (width 0.4) (layer "B.Cu") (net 8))
 (segment (start 121.92 68.58) (end 121.92 71.12) (width 0.4) (layer "B.Cu") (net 8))
 (segment (start 121.92 76.2) (end 124.46 76.2) (width 0.4) (layer "B.Cu") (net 8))
 (segment (start 121.92 71.12) (end 121.92 76.2) (width 0.4) (layer "B.Cu") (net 8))
 (segment (start 124.46 78.74) (end 124.46 76.2) (width 0.4) (layer "B.Cu") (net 8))
 (segment (start 124.46 50.8) (end 124.46 55.88) (width 0.4) (layer "B.Cu") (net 8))
 (segment (start 116.84 83.82) (end 116.84 86.36) (width 0.4) (layer "B.Cu") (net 2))
 (segment (start 121.92 91.44) (end 121.92 86.36) (width 0.4) (layer "B.Cu") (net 2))
 (segment (start 121.92 86.36) (end 116.84 86.36) (width 0.4) (layer "B.Cu") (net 2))
 (segment (start 124.46 91.44) (end 121.92 91.44) (width 0.4) (layer "B.Cu") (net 2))
 (segment (start 124.46 86.36) (end 124.46 88.9) (width 0.4) (layer "B.Cu") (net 7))
 (segment (start 116.84 58.42) (end 116.84 60.96) (width 0.4) (layer "B.Cu") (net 46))
 (segment (start 116.84 60.96) (end 116.84 63.5) (width 0.4) (layer "B.Cu") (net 46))
 (segment (start 116.84 55.88) (end 120.65 55.88) (width 0.4) (layer "B.Cu") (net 45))
 (segment (start 115.57 81.915) (end 115.57 76.2) (width 0.4) (layer "B.Cu") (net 45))
 (segment (start 113.03 82.55) (end 111.76 83.82) (width 0.4) (layer "B.Cu") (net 45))
 (segment (start 114.935 82.55) (end 115.57 81.915) (width 0.4) (layer "B.Cu") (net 45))
 (segment (start 114.935 82.55) (end 113.03 82.55) (width 0.4) (layer "B.Cu") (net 45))
 (segment (start 120.65 76.2) (end 115.57 76.2) (width 0.4) (layer "B.Cu") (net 45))
 (segment (start 120.65 55.88) (end 120.65 76.2) (width 0.4) (layer "B.Cu") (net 45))
 (segment (start 119.38 91.44) (end 116.84 91.44) (width 0.4) (layer "B.Cu") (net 4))
 (segment (start 111.76 96.52) (end 113.03 95.25) (width 0.4) (layer "B.Cu") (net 4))
 (segment (start 119.38 95.25) (end 119.38 91.44) (width 0.4) (layer "B.Cu") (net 4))
 (segment (start 113.03 95.25) (end 119.38 95.25) (width 0.4) (layer "B.Cu") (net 4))
 (segment (start 124.46 93.98) (end 127 91.44) (width 0.4) (layer "B.Cu") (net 6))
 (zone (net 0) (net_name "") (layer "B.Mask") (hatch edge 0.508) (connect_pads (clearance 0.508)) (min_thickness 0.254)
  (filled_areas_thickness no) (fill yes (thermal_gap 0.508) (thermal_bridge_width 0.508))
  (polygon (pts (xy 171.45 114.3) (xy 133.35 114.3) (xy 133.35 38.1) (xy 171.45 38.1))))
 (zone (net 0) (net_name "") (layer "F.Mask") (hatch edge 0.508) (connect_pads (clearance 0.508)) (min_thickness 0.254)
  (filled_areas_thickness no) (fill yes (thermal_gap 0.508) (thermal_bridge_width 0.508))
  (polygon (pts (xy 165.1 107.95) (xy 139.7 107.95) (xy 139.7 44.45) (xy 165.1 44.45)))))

